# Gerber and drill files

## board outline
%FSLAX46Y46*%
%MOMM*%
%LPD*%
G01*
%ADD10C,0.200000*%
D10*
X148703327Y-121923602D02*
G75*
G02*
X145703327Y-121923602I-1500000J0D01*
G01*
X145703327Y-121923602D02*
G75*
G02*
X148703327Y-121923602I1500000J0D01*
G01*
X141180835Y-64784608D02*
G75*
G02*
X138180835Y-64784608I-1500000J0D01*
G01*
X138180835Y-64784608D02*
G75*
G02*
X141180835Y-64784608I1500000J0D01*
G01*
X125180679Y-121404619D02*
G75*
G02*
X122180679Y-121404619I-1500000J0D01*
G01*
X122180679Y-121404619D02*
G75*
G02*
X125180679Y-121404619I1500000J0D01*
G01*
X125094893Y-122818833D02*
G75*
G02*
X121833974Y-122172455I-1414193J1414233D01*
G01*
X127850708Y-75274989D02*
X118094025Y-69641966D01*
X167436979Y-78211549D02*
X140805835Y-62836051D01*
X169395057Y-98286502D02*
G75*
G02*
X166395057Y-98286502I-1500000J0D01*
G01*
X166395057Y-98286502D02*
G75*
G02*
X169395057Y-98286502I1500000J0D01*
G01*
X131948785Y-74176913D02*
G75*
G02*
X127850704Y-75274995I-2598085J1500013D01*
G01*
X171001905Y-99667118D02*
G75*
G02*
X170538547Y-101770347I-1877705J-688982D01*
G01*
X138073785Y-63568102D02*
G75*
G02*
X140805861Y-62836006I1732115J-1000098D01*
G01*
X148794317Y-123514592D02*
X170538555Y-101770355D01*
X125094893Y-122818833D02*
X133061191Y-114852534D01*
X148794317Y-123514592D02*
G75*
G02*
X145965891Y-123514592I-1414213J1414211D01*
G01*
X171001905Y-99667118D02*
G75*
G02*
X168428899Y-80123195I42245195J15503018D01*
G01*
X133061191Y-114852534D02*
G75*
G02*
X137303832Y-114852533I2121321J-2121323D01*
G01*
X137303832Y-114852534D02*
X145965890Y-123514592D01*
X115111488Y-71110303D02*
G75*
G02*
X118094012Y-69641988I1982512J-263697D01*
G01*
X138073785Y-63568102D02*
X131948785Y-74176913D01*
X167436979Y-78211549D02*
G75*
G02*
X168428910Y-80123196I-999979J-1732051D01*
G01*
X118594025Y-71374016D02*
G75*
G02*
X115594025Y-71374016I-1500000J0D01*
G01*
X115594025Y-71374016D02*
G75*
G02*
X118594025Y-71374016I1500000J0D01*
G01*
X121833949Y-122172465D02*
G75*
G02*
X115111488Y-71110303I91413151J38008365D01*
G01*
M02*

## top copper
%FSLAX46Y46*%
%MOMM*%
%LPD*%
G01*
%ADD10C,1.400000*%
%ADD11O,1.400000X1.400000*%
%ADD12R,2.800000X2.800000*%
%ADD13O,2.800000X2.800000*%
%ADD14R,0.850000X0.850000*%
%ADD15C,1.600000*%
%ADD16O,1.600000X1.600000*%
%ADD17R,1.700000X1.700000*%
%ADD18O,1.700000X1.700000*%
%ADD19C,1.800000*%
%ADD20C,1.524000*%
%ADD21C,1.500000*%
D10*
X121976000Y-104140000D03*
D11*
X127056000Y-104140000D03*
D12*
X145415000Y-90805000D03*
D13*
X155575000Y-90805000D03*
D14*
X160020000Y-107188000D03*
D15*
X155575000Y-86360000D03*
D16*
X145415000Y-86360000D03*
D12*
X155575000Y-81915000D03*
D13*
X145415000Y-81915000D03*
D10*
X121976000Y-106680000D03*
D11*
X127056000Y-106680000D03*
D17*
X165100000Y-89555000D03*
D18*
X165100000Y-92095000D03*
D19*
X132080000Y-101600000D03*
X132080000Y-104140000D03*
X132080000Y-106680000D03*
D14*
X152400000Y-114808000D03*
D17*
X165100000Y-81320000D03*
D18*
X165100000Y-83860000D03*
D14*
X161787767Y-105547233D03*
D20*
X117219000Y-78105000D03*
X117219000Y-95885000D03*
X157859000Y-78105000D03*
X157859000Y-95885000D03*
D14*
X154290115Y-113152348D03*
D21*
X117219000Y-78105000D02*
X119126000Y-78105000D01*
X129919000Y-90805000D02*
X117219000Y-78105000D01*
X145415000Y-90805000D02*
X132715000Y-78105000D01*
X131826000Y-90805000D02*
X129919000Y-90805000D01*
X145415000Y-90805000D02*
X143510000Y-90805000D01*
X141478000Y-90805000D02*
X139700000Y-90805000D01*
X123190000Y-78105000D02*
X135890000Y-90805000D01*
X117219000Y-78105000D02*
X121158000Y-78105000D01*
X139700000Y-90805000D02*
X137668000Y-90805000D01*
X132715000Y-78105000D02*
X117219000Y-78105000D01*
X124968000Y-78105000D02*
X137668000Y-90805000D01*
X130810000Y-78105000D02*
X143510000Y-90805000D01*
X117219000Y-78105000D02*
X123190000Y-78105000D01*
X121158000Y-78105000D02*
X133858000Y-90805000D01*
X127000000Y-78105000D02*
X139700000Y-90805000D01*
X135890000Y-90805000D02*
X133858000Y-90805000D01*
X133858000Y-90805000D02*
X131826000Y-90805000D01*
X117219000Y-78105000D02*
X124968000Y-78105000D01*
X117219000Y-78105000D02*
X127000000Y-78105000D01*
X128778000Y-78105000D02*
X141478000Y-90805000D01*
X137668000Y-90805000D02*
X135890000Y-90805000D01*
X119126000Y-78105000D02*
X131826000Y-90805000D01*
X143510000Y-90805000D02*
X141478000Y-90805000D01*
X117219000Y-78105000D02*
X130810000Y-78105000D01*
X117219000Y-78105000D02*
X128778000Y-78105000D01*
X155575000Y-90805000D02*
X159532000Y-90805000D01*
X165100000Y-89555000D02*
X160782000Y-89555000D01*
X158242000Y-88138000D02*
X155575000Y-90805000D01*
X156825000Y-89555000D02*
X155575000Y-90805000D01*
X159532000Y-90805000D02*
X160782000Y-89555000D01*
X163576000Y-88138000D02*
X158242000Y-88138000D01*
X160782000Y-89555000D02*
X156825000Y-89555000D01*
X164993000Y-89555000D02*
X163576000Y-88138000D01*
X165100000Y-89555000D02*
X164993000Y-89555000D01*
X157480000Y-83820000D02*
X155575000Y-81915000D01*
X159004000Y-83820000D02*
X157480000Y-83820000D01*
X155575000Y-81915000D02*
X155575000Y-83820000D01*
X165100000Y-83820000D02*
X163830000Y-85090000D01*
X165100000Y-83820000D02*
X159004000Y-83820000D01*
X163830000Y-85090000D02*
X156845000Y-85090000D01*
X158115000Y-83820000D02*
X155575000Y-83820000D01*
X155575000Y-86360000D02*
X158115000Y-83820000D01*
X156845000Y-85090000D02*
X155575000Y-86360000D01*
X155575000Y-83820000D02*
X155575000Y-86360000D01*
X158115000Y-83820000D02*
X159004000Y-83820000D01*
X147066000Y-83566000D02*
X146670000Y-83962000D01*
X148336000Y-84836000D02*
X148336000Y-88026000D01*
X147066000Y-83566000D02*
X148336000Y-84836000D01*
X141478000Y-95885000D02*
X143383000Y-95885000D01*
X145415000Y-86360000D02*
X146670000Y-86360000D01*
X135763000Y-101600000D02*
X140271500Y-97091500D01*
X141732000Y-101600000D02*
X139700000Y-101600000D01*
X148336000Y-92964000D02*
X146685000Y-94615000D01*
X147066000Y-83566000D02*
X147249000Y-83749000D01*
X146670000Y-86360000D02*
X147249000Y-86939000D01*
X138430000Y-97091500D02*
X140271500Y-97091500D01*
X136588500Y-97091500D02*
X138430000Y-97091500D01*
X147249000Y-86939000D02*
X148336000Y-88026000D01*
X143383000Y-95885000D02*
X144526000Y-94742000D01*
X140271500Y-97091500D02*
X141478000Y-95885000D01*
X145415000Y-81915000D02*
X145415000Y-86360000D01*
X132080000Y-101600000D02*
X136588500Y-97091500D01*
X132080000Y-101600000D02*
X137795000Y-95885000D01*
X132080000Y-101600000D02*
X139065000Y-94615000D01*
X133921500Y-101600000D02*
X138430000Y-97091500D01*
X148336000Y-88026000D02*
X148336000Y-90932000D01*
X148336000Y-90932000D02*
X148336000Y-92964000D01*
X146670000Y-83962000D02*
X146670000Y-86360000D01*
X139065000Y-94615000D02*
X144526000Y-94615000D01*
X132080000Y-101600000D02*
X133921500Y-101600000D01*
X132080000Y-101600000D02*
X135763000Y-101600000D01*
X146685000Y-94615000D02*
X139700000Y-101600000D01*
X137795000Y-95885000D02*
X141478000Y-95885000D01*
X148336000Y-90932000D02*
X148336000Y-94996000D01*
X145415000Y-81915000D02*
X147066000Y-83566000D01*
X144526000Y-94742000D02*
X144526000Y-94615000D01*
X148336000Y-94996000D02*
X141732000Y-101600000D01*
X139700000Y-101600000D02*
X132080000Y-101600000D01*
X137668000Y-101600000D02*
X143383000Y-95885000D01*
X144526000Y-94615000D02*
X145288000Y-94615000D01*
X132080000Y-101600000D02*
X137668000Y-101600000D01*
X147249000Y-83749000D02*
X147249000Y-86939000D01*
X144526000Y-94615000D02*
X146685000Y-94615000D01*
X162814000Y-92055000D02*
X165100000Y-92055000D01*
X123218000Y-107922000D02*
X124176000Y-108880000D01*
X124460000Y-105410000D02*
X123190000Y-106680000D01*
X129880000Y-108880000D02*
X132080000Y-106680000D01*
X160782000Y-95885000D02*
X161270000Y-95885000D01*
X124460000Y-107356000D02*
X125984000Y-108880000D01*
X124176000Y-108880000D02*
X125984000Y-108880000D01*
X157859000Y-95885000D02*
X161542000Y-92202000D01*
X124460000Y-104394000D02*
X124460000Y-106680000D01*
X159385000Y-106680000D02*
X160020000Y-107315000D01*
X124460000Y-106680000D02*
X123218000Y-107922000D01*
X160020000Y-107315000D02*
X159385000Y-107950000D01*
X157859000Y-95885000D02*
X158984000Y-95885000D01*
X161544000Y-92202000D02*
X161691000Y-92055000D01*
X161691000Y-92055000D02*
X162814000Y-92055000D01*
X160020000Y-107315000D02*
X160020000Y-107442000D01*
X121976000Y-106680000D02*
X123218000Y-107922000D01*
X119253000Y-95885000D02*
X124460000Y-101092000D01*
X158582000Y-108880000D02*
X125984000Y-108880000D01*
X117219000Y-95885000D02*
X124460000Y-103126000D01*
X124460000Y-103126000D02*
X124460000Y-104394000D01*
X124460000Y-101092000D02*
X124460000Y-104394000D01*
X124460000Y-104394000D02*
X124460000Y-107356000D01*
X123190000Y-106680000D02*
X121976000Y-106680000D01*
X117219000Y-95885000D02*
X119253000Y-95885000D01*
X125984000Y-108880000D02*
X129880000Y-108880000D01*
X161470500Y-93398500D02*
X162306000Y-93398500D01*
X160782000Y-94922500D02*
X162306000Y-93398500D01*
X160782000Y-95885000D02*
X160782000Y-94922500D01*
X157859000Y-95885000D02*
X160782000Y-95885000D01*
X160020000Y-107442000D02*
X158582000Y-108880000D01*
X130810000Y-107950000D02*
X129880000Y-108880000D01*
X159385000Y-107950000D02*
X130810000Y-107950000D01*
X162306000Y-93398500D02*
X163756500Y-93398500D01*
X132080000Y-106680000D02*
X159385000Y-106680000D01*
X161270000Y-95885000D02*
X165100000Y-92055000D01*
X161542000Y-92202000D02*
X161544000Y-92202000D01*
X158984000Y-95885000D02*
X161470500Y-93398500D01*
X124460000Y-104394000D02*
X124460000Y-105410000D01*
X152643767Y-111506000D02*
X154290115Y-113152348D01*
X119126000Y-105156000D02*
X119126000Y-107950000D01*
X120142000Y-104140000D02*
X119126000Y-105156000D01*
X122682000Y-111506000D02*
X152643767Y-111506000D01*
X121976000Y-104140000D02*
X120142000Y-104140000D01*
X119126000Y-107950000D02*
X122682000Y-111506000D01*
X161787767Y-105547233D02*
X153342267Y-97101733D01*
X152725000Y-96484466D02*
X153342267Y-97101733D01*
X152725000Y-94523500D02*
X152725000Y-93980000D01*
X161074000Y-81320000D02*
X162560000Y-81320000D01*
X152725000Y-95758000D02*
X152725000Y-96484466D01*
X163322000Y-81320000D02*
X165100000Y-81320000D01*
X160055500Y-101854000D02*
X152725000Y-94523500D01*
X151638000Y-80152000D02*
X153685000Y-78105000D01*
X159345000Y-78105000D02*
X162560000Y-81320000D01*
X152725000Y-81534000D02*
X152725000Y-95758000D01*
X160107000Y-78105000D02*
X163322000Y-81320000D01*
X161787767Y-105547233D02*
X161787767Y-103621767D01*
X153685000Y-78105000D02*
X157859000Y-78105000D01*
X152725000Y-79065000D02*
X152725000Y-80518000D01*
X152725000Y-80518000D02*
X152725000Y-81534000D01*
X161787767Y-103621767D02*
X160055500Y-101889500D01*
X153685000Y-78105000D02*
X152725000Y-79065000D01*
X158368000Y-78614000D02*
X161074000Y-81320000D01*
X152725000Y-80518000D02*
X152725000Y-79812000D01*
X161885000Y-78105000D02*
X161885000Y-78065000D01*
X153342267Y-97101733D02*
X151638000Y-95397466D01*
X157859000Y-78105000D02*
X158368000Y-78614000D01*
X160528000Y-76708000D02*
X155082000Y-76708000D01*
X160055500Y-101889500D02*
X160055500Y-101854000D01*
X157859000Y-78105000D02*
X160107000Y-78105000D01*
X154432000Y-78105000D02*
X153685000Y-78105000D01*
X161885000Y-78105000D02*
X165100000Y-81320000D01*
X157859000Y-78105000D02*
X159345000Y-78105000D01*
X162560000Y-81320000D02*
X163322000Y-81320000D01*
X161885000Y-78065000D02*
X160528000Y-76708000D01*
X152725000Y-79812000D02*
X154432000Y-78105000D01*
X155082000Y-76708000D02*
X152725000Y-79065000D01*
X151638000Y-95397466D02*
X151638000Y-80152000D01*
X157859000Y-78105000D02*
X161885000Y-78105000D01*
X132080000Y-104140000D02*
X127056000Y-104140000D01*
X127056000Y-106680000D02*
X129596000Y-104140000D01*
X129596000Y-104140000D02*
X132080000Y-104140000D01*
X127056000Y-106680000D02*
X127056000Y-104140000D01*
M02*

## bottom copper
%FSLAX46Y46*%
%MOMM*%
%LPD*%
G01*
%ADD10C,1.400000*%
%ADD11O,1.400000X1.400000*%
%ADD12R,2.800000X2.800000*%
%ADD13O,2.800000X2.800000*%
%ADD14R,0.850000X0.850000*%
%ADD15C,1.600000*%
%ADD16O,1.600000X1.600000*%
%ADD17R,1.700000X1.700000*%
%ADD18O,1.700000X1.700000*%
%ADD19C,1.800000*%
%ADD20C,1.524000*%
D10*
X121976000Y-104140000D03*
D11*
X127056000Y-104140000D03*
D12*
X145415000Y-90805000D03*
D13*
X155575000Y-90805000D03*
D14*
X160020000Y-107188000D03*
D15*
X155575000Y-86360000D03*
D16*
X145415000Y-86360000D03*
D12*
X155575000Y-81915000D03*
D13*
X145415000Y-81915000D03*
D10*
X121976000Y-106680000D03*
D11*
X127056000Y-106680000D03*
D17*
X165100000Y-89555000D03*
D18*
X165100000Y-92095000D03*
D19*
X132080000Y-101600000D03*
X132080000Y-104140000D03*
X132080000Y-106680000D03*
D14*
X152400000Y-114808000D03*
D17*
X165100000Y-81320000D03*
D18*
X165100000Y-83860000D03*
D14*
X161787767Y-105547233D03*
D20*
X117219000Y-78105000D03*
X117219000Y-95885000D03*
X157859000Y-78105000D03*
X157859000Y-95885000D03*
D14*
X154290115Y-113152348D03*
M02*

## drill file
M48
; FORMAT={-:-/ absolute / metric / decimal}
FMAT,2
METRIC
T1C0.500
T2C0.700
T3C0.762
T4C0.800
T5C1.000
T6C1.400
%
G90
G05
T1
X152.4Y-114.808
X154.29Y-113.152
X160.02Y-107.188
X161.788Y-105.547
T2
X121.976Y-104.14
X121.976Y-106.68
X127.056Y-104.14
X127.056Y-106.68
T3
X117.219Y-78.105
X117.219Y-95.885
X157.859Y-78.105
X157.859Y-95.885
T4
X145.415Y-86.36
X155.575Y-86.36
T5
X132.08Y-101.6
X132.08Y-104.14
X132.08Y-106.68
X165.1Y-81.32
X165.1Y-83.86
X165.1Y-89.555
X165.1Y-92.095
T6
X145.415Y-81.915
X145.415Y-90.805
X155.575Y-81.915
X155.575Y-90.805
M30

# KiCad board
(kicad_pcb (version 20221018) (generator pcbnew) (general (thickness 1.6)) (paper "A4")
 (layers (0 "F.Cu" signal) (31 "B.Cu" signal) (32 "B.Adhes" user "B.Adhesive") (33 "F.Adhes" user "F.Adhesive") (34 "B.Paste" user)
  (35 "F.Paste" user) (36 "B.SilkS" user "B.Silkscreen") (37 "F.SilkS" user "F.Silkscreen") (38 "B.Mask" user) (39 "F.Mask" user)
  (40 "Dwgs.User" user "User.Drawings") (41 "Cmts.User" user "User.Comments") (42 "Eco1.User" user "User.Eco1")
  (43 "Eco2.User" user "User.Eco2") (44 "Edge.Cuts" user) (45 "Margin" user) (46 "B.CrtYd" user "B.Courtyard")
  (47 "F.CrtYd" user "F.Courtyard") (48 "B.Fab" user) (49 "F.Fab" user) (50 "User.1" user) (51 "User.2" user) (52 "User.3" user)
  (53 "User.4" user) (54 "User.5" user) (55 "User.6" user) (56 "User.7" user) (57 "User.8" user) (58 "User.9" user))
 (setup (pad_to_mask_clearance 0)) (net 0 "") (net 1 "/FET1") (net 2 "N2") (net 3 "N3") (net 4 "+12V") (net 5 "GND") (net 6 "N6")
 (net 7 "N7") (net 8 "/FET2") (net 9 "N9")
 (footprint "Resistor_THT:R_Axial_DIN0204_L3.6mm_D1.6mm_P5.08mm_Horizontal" (layer "F.Cu") (at 121.976 104.14)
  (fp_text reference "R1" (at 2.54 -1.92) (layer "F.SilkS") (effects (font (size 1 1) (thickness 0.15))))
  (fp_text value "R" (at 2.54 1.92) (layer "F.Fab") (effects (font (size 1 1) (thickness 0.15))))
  (pad "1" thru_hole circle (at 0 0) (size 1.4 1.4) (drill 0.7) (layers "*.Cu" "*.Mask") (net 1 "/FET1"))
  (pad "2" thru_hole oval (at 5.08 0) (size 1.4 1.4) (drill 0.7) (layers "*.Cu" "*.Mask") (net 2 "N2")))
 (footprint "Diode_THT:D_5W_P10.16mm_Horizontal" (layer "F.Cu") (at 145.415 90.805)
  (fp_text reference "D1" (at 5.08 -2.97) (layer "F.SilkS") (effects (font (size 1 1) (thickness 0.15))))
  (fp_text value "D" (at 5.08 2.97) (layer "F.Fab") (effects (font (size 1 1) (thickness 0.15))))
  (pad "1" thru_hole rect (at 0 0) (size 2.8 2.8) (drill 1.4) (layers "*.Cu" "*.Mask") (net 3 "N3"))
  (pad "2" thru_hole oval (at 10.16 0) (size 2.8 2.8) (drill 1.4) (layers "*.Cu" "*.Mask") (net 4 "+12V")))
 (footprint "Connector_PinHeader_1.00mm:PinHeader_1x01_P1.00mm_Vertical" (layer "F.Cu") (at 160.02 107.188)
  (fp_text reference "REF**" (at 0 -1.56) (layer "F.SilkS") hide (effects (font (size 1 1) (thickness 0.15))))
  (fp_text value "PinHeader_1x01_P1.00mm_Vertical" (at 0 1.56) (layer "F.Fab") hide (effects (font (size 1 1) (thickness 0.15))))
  (pad "1" thru_hole rect (at 0 0) (size 0.85 0.85) (drill 0.5) (layers "*.Cu" "*.Mask") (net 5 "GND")))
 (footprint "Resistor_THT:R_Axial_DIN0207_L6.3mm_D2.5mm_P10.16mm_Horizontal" (layer "F.Cu") (at 155.575 86.36 180)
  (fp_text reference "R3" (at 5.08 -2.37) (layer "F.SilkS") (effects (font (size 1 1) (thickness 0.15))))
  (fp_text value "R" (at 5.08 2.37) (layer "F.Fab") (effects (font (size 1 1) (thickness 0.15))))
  (pad "1" thru_hole circle (at 0 0 180) (size 1.6 1.6) (drill 0.8) (layers "*.Cu" "*.Mask") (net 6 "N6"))
  (pad "2" thru_hole oval (at 10.16 0 180) (size 1.6 1.6) (drill 0.8) (layers "*.Cu" "*.Mask") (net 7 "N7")))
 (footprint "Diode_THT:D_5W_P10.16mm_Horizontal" (layer "F.Cu") (at 155.575 81.915 180)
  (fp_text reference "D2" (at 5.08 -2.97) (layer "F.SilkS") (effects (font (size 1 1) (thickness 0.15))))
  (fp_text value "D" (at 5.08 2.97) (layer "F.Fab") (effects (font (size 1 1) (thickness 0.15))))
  (pad "1" thru_hole rect (at 0 0 180) (size 2.8 2.8) (drill 1.4) (layers "*.Cu" "*.Mask") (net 6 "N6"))
  (pad "2" thru_hole oval (at 10.16 0 180) (size 2.8 2.8) (drill 1.4) (layers "*.Cu" "*.Mask") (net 7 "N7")))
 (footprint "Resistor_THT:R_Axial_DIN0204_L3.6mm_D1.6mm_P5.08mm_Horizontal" (layer "F.Cu") (at 121.976 106.68)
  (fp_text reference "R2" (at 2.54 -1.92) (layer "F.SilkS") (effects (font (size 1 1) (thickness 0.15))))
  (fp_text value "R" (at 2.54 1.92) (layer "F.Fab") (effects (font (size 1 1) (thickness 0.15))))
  (pad "1" thru_hole circle (at 0 0) (size 1.4 1.4) (drill 0.7) (layers "*.Cu" "*.Mask") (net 5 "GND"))
  (pad "2" thru_hole oval (at 5.08 0) (size 1.4 1.4) (drill 0.7) (layers "*.Cu" "*.Mask") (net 2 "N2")))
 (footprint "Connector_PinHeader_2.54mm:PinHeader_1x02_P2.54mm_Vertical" (layer "F.Cu") (at 165.1 89.555)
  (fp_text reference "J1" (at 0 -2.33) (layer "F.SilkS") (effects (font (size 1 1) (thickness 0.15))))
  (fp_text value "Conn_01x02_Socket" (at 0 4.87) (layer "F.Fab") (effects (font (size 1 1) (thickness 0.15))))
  (pad "1" thru_hole rect (at 0 0) (size 1.7 1.7) (drill 1) (layers "*.Cu" "*.Mask") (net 4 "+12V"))
  (pad "2" thru_hole oval (at 0 2.54) (size 1.7 1.7) (drill 1) (layers "*.Cu" "*.Mask") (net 5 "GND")))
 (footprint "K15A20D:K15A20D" (layer "F.Cu") (at 154.432 104.14 -90)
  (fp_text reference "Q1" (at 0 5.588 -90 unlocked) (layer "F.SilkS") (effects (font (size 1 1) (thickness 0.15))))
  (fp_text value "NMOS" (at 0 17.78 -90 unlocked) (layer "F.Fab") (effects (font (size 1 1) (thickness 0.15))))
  (pad "1" thru_hole circle (at -2.54 22.352 90) (size 1.8 1.8) (drill 1) (layers "*.Cu" "*.Mask") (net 7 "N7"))
  (pad "2" thru_hole circle (at 0 22.352 90) (size 1.8 1.8) (drill 1) (layers "*.Cu" "*.Mask") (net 2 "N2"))
  (pad "3" thru_hole circle (at 2.54 22.352 90) (size 1.8 1.8) (drill 1) (layers "*.Cu" "*.Mask") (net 5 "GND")))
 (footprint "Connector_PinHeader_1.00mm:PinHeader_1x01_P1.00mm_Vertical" (layer "F.Cu") (at 152.4 114.808)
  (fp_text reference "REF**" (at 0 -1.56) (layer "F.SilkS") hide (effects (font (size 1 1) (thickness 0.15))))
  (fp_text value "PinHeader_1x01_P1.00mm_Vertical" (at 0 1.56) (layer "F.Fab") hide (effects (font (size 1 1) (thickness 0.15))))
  (pad "1" thru_hole rect (at 0 0) (size 0.85 0.85) (drill 0.5) (layers "*.Cu" "*.Mask") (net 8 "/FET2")))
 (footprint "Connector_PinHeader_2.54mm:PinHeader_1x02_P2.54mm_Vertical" (layer "F.Cu") (at 165.1 81.32)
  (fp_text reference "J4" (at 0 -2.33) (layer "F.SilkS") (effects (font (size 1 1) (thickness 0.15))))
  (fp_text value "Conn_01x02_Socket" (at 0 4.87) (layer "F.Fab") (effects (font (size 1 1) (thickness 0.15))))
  (pad "1" thru_hole rect (at 0 0) (size 1.7 1.7) (drill 1) (layers "*.Cu" "*.Mask") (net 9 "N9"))
  (pad "2" thru_hole oval (at 0 2.54) (size 1.7 1.7) (drill 1) (layers "*.Cu" "*.Mask") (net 6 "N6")))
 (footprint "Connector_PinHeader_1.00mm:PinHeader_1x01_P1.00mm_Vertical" (layer "F.Cu") (at 161.787767 105.547233)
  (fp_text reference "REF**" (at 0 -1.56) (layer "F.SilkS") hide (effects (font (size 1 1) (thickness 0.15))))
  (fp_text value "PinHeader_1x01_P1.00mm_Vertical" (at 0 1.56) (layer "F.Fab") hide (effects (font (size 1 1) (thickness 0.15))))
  (pad "1" thru_hole rect (at 0 0) (size 0.85 0.85) (drill 0.5) (layers "*.Cu" "*.Mask") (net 9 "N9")))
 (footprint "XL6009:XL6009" (layer "F.Cu") (at 112.139 86.995 90)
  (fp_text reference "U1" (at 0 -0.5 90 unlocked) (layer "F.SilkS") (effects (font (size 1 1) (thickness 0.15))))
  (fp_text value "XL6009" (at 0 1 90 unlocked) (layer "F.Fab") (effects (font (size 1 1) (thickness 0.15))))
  (pad "1" thru_hole circle (at 8.89 5.08 90) (size 1.524 1.524) (drill 0.762) (layers "*.Cu" "*.Mask") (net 3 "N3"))
  (pad "2" thru_hole circle (at -8.89 5.08 90) (size 1.524 1.524) (drill 0.762) (layers "*.Cu" "*.Mask") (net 5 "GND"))
  (pad "3" thru_hole circle (at 8.89 45.72 90) (size 1.524 1.524) (drill 0.762) (layers "*.Cu" "*.Mask") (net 9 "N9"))
  (pad "4" thru_hole circle (at -8.89 45.72 90) (size 1.524 1.524) (drill 0.762) (layers "*.Cu" "*.Mask") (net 5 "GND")))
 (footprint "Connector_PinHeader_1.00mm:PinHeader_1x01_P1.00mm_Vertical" (layer "F.Cu") (at 154.290115 113.152348)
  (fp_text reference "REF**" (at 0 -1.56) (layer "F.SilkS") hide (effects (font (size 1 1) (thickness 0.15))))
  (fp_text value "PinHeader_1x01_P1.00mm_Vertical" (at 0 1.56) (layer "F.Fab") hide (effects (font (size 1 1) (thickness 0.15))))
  (pad "1" thru_hole rect (at 0 0) (size 0.85 0.85) (drill 0.5) (layers "*.Cu" "*.Mask") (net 1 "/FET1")))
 (gr_circle (center 147.203327 121.923602) (end 145.703327 121.923602) (stroke (width 0.2) (type solid)) (fill none) (layer "Edge.Cuts"))
 (gr_circle (center 139.680835 64.784608) (end 138.180835 64.784608) (stroke (width 0.2) (type solid)) (fill none) (layer "Edge.Cuts"))
 (gr_circle (center 123.680679 121.404619) (end 122.180679 121.404619) (stroke (width 0.2) (type solid)) (fill none) (layer "Edge.Cuts"))
 (gr_arc (start 125.094893 122.818833) (mid 123.291827 123.366429) (end 121.833949 122.172465) (stroke (width 0.2) (type solid))
  (layer "Edge.Cuts"))
 (gr_line (start 127.850708 75.274989) (end 118.094025 69.641966) (stroke (width 0.2) (type solid)) (layer "Edge.Cuts"))
 (gr_line (start 167.436979 78.211549) (end 140.805835 62.836051) (stroke (width 0.2) (type solid)) (layer "Edge.Cuts"))
 (gr_circle (center 167.895057 98.286502) (end 166.395057 98.286502) (stroke (width 0.2) (type solid)) (fill none) (layer "Edge.Cuts"))
 (gr_arc (start 131.948785 74.176913) (mid 130.127164 75.57469) (end 127.850708 75.274989) (stroke (width 0.2) (type solid))
  (layer "Edge.Cuts"))
 (gr_arc (start 171.001905 99.667118) (mid 171.077482 100.78642) (end 170.538555 101.770355) (stroke (width 0.2) (type solid))
  (layer "Edge.Cuts"))
 (gr_arc (start 138.073785 63.568102) (mid 139.288193 62.636273) (end 140.805835 62.836051) (stroke (width 0.2) (type solid))
  (layer "Edge.Cuts"))
 (gr_line (start 148.794317 123.514592) (end 170.538555 101.770355) (stroke (width 0.2) (type solid)) (layer "Edge.Cuts"))
 (gr_line (start 125.094893 122.818833) (end 133.061191 114.852534) (stroke (width 0.2) (type solid)) (layer "Edge.Cuts"))
 (gr_arc (start 148.794317 123.514592) (mid 147.380103 124.100379) (end 145.96589 123.514592) (stroke (width 0.2) (type solid))
  (layer "Edge.Cuts"))
 (gr_arc (start 171.001905 99.667118) (mid 168.632081 90.037778) (end 168.428899 80.123195) (stroke (width 0.2) (type solid))
  (layer "Edge.Cuts"))
 (gr_arc (start 133.061191 114.852534) (mid 135.182511 113.973855) (end 137.303832 114.852534) (stroke (width 0.2) (type solid))
  (layer "Edge.Cuts"))
 (gr_line (start 137.303832 114.852534) (end 145.96589 123.514592) (stroke (width 0.2) (type solid)) (layer "Edge.Cuts"))
 (gr_arc (start 115.111488 71.110303) (mid 116.210646 69.579682) (end 118.094025 69.641966) (stroke (width 0.2) (type solid))
  (layer "Edge.Cuts"))
 (gr_line (start 138.073785 63.568102) (end 131.948785 74.176913) (stroke (width 0.2) (type solid)) (layer "Edge.Cuts"))
 (gr_arc (start 167.436979 78.211549) (mid 168.212232 79.022454) (end 168.428899 80.123195) (stroke (width 0.2) (type solid))
  (layer "Edge.Cuts"))
 (gr_circle (center 117.094025 71.374016) (end 115.594025 71.374016) (stroke (width 0.2) (type solid)) (fill none) (layer "Edge.Cuts"))
 (gr_arc (start 121.833949 122.172465) (mid 115.094059 97.086193) (end 115.111488 71.110303) (stroke (width 0.2) (type solid))
  (layer "Edge.Cuts"))
 (segment (start 117.219 78.105) (end 119.126 78.105) (width 1.5) (layer "F.Cu") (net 3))
 (segment (start 129.919 90.805) (end 117.219 78.105) (width 1.5) (layer "F.Cu") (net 3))
 (segment (start 145.415 90.805) (end 132.715 78.105) (width 1.5) (layer "F.Cu") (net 3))
 (segment (start 131.826 90.805) (end 129.919 90.805) (width 1.5) (layer "F.Cu") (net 3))
 (segment (start 145.415 90.805) (end 143.51 90.805) (width 1.5) (layer "F.Cu") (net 3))
 (segment (start 141.478 90.805) (end 139.7 90.805) (width 1.5) (layer "F.Cu") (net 3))
 (segment (start 123.19 78.105) (end 135.89 90.805) (width 1.5) (layer "F.Cu") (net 3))
 (segment (start 117.219 78.105) (end 121.158 78.105) (width 1.5) (layer "F.Cu") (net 3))
 (segment (start 139.7 90.805) (end 137.668 90.805) (width 1.5) (layer "F.Cu") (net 3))
 (segment (start 132.715 78.105) (end 117.219 78.105) (width 1.5) (layer "F.Cu") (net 3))
 (segment (start 124.968 78.105) (end 137.668 90.805) (width 1.5) (layer "F.Cu") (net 3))
 (segment (start 130.81 78.105) (end 143.51 90.805) (width 1.5) (layer "F.Cu") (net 3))
 (segment (start 117.219 78.105) (end 123.19 78.105) (width 1.5) (layer "F.Cu") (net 3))
 (segment (start 121.158 78.105) (end 133.858 90.805) (width 1.5) (layer "F.Cu") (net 3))
 (segment (start 127 78.105) (end 139.7 90.805) (width 1.5) (layer "F.Cu") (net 3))
 (segment (start 135.89 90.805) (end 133.858 90.805) (width 1.5) (layer "F.Cu") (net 3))
 (segment (start 133.858 90.805) (end 131.826 90.805) (width 1.5) (layer "F.Cu") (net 3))
 (segment (start 117.219 78.105) (end 124.968 78.105) (width 1.5) (layer "F.Cu") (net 3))
 (segment (start 117.219 78.105) (end 127 78.105) (width 1.5) (layer "F.Cu") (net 3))
 (segment (start 128.778 78.105) (end 141.478 90.805) (width 1.5) (layer "F.Cu") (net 3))
 (segment (start 137.668 90.805) (end 135.89 90.805) (width 1.5) (layer "F.Cu") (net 3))
 (segment (start 119.126 78.105) (end 131.826 90.805) (width 1.5) (layer "F.Cu") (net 3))
 (segment (start 143.51 90.805) (end 141.478 90.805) (width 1.5) (layer "F.Cu") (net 3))
 (segment (start 117.219 78.105) (end 130.81 78.105) (width 1.5) (layer "F.Cu") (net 3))
 (segment (start 117.219 78.105) (end 128.778 78.105) (width 1.5) (layer "F.Cu") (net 3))
 (segment (start 155.575 90.805) (end 159.532 90.805) (width 1.5) (layer "F.Cu") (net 4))
 (segment (start 165.1 89.555) (end 160.782 89.555) (width 1.5) (layer "F.Cu") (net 4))
 (segment (start 158.242 88.138) (end 155.575 90.805) (width 1.5) (layer "F.Cu") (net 4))
 (segment (start 156.825 89.555) (end 155.575 90.805) (width 1.5) (layer "F.Cu") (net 4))
 (segment (start 159.532 90.805) (end 160.782 89.555) (width 1.5) (layer "F.Cu") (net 4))
 (segment (start 163.576 88.138) (end 158.242 88.138) (width 1.5) (layer "F.Cu") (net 4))
 (segment (start 160.782 89.555) (end 156.825 89.555) (width 1.5) (layer "F.Cu") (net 4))
 (segment (start 164.993 89.555) (end 163.576 88.138) (width 1.5) (layer "F.Cu") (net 4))
 (segment (start 165.1 89.555) (end 164.993 89.555) (width 1.5) (layer "F.Cu") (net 4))
 (segment (start 157.48 83.82) (end 155.575 81.915) (width 1.5) (layer "F.Cu") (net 6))
 (segment (start 159.004 83.82) (end 157.48 83.82) (width 1.5) (layer "F.Cu") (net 6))
 (segment (start 155.575 81.915) (end 155.575 83.82) (width 1.5) (layer "F.Cu") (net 6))
 (segment (start 165.1 83.82) (end 163.83 85.09) (width 1.5) (layer "F.Cu") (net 6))
 (segment (start 165.1 83.82) (end 159.004 83.82) (width 1.5) (layer "F.Cu") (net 6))
 (segment (start 163.83 85.09) (end 156.845 85.09) (width 1.5) (layer "F.Cu") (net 6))
 (segment (start 158.115 83.82) (end 155.575 83.82) (width 1.5) (layer "F.Cu") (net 6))
 (segment (start 155.575 86.36) (end 158.115 83.82) (width 1.5) (layer "F.Cu") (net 6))
 (segment (start 156.845 85.09) (end 155.575 86.36) (width 1.5) (layer "F.Cu") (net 6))
 (segment (start 155.575 83.82) (end 155.575 86.36) (width 1.5) (layer "F.Cu") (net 6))
 (segment (start 158.115 83.82) (end 159.004 83.82) (width 1.5) (layer "F.Cu") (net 6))
 (segment (start 147.066 83.566) (end 146.67 83.962) (width 1.5) (layer "F.Cu") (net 7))
 (segment (start 148.336 84.836) (end 148.336 88.026) (width 1.5) (layer "F.Cu") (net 7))
 (segment (start 147.066 83.566) (end 148.336 84.836) (width 1.5) (layer "F.Cu") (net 7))
 (segment (start 141.478 95.885) (end 143.383 95.885) (width 1.5) (layer "F.Cu") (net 7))
 (segment (start 145.415 86.36) (end 146.67 86.36) (width 1.5) (layer "F.Cu") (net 7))
 (segment (start 135.763 101.6) (end 140.2715 97.0915) (width 1.5) (layer "F.Cu") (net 7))
 (segment (start 141.732 101.6) (end 139.7 101.6) (width 1.5) (layer "F.Cu") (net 7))
 (segment (start 148.336 92.964) (end 146.685 94.615) (width 1.5) (layer "F.Cu") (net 7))
 (segment (start 147.066 83.566) (end 147.249 83.749) (width 1.5) (layer "F.Cu") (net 7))
 (segment (start 146.67 86.36) (end 147.249 86.939) (width 1.5) (layer "F.Cu") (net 7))
 (segment (start 138.43 97.0915) (end 140.2715 97.0915) (width 1.5) (layer "F.Cu") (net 7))
 (segment (start 136.5885 97.0915) (end 138.43 97.0915) (width 1.5) (layer "F.Cu") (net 7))
 (segment (start 147.249 86.939) (end 148.336 88.026) (width 1.5) (layer "F.Cu") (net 7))
 (segment (start 143.383 95.885) (end 144.526 94.742) (width 1.5) (layer "F.Cu") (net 7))
 (segment (start 140.2715 97.0915) (end 141.478 95.885) (width 1.5) (layer "F.Cu") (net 7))
 (segment (start 145.415 81.915) (end 145.415 86.36) (width 1.5) (layer "F.Cu") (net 7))
 (segment (start 132.08 101.6) (end 136.5885 97.0915) (width 1.5) (layer "F.Cu") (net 7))
 (segment (start 132.08 101.6) (end 137.795 95.885) (width 1.5) (layer "F.Cu") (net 7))
 (segment (start 132.08 101.6) (end 139.065 94.615) (width 1.5) (layer "F.Cu") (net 7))
 (segment (start 133.9215 101.6) (end 138.43 97.0915) (width 1.5) (layer "F.Cu") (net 7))
 (segment (start 148.336 88.026) (end 148.336 90.932) (width 1.5) (layer "F.Cu") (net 7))
 (segment (start 148.336 90.932) (end 148.336 92.964) (width 1.5) (layer "F.Cu") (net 7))
 (segment (start 146.67 83.962) (end 146.67 86.36) (width 1.5) (layer "F.Cu") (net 7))
 (segment (start 139.065 94.615) (end 144.526 94.615) (width 1.5) (layer "F.Cu") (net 7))
 (segment (start 132.08 101.6) (end 133.9215 101.6) (width 1.5) (layer "F.Cu") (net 7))
 (segment (start 132.08 101.6) (end 135.763 101.6) (width 1.5) (layer "F.Cu") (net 7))
 (segment (start 146.685 94.615) (end 139.7 101.6) (width 1.5) (layer "F.Cu") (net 7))
 (segment (start 137.795 95.885) (end 141.478 95.885) (width 1.5) (layer "F.Cu") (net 7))
 (segment (start 148.336 90.932) (end 148.336 94.996) (width 1.5) (layer "F.Cu") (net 7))
 (segment (start 145.415 81.915) (end 147.066 83.566) (width 1.5) (layer "F.Cu") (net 7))
 (segment (start 144.526 94.742) (end 144.526 94.615) (width 1.5) (layer "F.Cu") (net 7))
 (segment (start 148.336 94.996) (end 141.732 101.6) (width 1.5) (layer "F.Cu") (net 7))
 (segment (start 139.7 101.6) (end 132.08 101.6) (width 1.5) (layer "F.Cu") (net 7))
 (segment (start 137.668 101.6) (end 143.383 95.885) (width 1.5) (layer "F.Cu") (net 7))
 (segment (start 144.526 94.615) (end 145.288 94.615) (width 1.5) (layer "F.Cu") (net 7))
 (segment (start 132.08 101.6) (end 137.668 101.6) (width 1.5) (layer "F.Cu") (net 7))
 (segment (start 147.249 83.749) (end 147.249 86.939) (width 1.5) (layer "F.Cu") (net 7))
 (segment (start 144.526 94.615) (end 146.685 94.615) (width 1.5) (layer "F.Cu") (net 7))
 (segment (start 162.814 92.055) (end 165.1 92.055) (width 1.5) (layer "F.Cu") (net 5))
 (segment (start 123.218 107.922) (end 124.176 108.88) (width 1.5) (layer "F.Cu") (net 5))
 (segment (start 124.46 105.41) (end 123.19 106.68) (width 1.5) (layer "F.Cu") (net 5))
 (segment (start 129.88 108.88) (end 132.08 106.68) (width 1.5) (layer "F.Cu") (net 5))
 (segment (start 160.782 95.885) (end 161.27 95.885) (width 1.5) (layer "F.Cu") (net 5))
 (segment (start 124.46 107.356) (end 125.984 108.88) (width 1.5) (layer "F.Cu") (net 5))
 (segment (start 124.176 108.88) (end 125.984 108.88) (width 1.5) (layer "F.Cu") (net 5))
 (segment (start 157.859 95.885) (end 161.542 92.202) (width 1.5) (layer "F.Cu") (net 5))
 (segment (start 124.46 104.394) (end 124.46 106.68) (width 1.5) (layer "F.Cu") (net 5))
 (segment (start 159.385 106.68) (end 160.02 107.315) (width 1.5) (layer "F.Cu") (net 5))
 (segment (start 124.46 106.68) (end 123.218 107.922) (width 1.5) (layer "F.Cu") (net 5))
 (segment (start 160.02 107.315) (end 159.385 107.95) (width 1.5) (layer "F.Cu") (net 5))
 (segment (start 157.859 95.885) (end 158.984 95.885) (width 1.5) (layer "F.Cu") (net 5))
 (segment (start 161.544 92.202) (end 161.691 92.055) (width 1.5) (layer "F.Cu") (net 5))
 (segment (start 161.691 92.055) (end 162.814 92.055) (width 1.5) (layer "F.Cu") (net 5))
 (segment (start 160.02 107.315) (end 160.02 107.442) (width 1.5) (layer "F.Cu") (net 5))
 (segment (start 121.976 106.68) (end 123.218 107.922) (width 1.5) (layer "F.Cu") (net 5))
 (segment (start 119.253 95.885) (end 124.46 101.092) (width 1.5) (layer "F.Cu") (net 5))
 (segment (start 158.582 108.88) (end 125.984 108.88) (width 1.5) (layer "F.Cu") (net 5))
 (segment (start 117.219 95.885) (end 124.46 103.126) (width 1.5) (layer "F.Cu") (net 5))
 (segment (start 124.46 103.126) (end 124.46 104.394) (width 1.5) (layer "F.Cu") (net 5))
 (segment (start 124.46 101.092) (end 124.46 104.394) (width 1.5) (layer "F.Cu") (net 5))
 (segment (start 124.46 104.394) (end 124.46 107.356) (width 1.5) (layer "F.Cu") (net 5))
 (segment (start 123.19 106.68) (end 121.976 106.68) (width 1.5) (layer "F.Cu") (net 5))
 (segment (start 117.219 95.885) (end 119.253 95.885) (width 1.5) (layer "F.Cu") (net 5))
 (segment (start 125.984 108.88) (end 129.88 108.88) (width 1.5) (layer "F.Cu") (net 5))
 (segment (start 161.4705 93.3985) (end 162.306 93.3985) (width 1.5) (layer "F.Cu") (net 5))
 (segment (start 160.782 94.9225) (end 162.306 93.3985) (width 1.5) (layer "F.Cu") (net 5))
 (segment (start 160.782 95.885) (end 160.782 94.9225) (width 1.5) (layer "F.Cu") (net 5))
 (segment (start 157.859 95.885) (end 160.782 95.885) (width 1.5) (layer "F.Cu") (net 5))
 (segment (start 160.02 107.442) (end 158.582 108.88) (width 1.5) (layer "F.Cu") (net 5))
 (segment (start 130.81 107.95) (end 129.88 108.88) (width 1.5) (layer "F.Cu") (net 5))
 (segment (start 159.385 107.95) (end 130.81 107.95) (width 1.5) (layer "F.Cu") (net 5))
 (segment (start 162.306 93.3985) (end 163.7565 93.3985) (width 1.5) (layer "F.Cu") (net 5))
 (segment (start 132.08 106.68) (end 159.385 106.68) (width 1.5) (layer "F.Cu") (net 5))
 (segment (start 161.27 95.885) (end 165.1 92.055) (width 1.5) (layer "F.Cu") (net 5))
 (segment (start 161.542 92.202) (end 161.544 92.202) (width 1.5) (layer "F.Cu") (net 5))
 (segment (start 158.984 95.885) (end 161.4705 93.3985) (width 1.5) (layer "F.Cu") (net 5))
 (segment (start 124.46 104.394) (end 124.46 105.41) (width 1.5) (layer "F.Cu") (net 5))
 (segment (start 152.643767 111.506) (end 154.290115 113.152348) (width 1.5) (layer "F.Cu") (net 1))
 (segment (start 119.126 105.156) (end 119.126 107.95) (width 1.5) (layer "F.Cu") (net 1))
 (segment (start 120.142 104.14) (end 119.126 105.156) (width 1.5) (layer "F.Cu") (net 1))
 (segment (start 122.682 111.506) (end 152.643767 111.506) (width 1.5) (layer "F.Cu") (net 1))
 (segment (start 121.976 104.14) (end 120.142 104.14) (width 1.5) (layer "F.Cu") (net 1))
 (segment (start 119.126 107.95) (end 122.682 111.506) (width 1.5) (layer "F.Cu") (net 1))
 (segment (start 161.787767 105.547233) (end 153.342267 97.101733) (width 1.5) (layer "F.Cu") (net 9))
 (segment (start 152.725 96.484466) (end 153.342267 97.101733) (width 1.5) (layer "F.Cu") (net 9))
 (segment (start 152.725 94.5235) (end 152.725 93.98) (width 1.5) (layer "F.Cu") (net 9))
 (segment (start 161.074 81.32) (end 162.56 81.32) (width 1.5) (layer "F.Cu") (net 9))
 (segment (start 152.725 95.758) (end 152.725 96.484466) (width 1.5) (layer "F.Cu") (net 9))
 (segment (start 163.322 81.32) (end 165.1 81.32) (width 1.5) (layer "F.Cu") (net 9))
 (segment (start 160.0555 101.854) (end 152.725 94.5235) (width 1.5) (layer "F.Cu") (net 9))
 (segment (start 151.638 80.152) (end 153.685 78.105) (width 1.5) (layer "F.Cu") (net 9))
 (segment (start 159.345 78.105) (end 162.56 81.32) (width 1.5) (layer "F.Cu") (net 9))
 (segment (start 152.725 81.534) (end 152.725 95.758) (width 1.5) (layer "F.Cu") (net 9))
 (segment (start 160.107 78.105) (end 163.322 81.32) (width 1.5) (layer "F.Cu") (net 9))
 (segment (start 161.787767 105.547233) (end 161.787767 103.621767) (width 1.5) (layer "F.Cu") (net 9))
 (segment (start 153.685 78.105) (end 157.859 78.105) (width 1.5) (layer "F.Cu") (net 9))
 (segment (start 152.725 79.065) (end 152.725 80.518) (width 1.5) (layer "F.Cu") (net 9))
 (segment (start 152.725 80.518) (end 152.725 81.534) (width 1.5) (layer "F.Cu") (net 9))
 (segment (start 161.787767 103.621767) (end 160.0555 101.8895) (width 1.5) (layer "F.Cu") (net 9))
 (segment (start 153.685 78.105) (end 152.725 79.065) (width 1.5) (layer "F.Cu") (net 9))
 (segment (start 158.368 78.614) (end 161.074 81.32) (width 1.5) (layer "F.Cu") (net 9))
 (segment (start 152.725 80.518) (end 152.725 79.812) (width 1.5) (layer "F.Cu") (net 9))
 (segment (start 161.885 78.105) (end 161.885 78.065) (width 1.5) (layer "F.Cu") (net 9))
 (segment (start 153.342267 97.101733) (end 151.638 95.397466) (width 1.5) (layer "F.Cu") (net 9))
 (segment (start 157.859 78.105) (end 158.368 78.614) (width 1.5) (layer "F.Cu") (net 9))
 (segment (start 160.528 76.708) (end 155.082 76.708) (width 1.5) (layer "F.Cu") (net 9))
 (segment (start 160.0555 101.8895) (end 160.0555 101.854) (width 1.5) (layer "F.Cu") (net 9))
 (segment (start 157.859 78.105) (end 160.107 78.105) (width 1.5) (layer "F.Cu") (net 9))
 (segment (start 154.432 78.105) (end 153.685 78.105) (width 1.5) (layer "F.Cu") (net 9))
 (segment (start 161.885 78.105) (end 165.1 81.32) (width 1.5) (layer "F.Cu") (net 9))
 (segment (start 157.859 78.105) (end 159.345 78.105) (width 1.5) (layer "F.Cu") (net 9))
 (segment (start 162.56 81.32) (end 163.322 81.32) (width 1.5) (layer "F.Cu") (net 9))
 (segment (start 161.885 78.065) (end 160.528 76.708) (width 1.5) (layer "F.Cu") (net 9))
 (segment (start 152.725 79.812) (end 154.432 78.105) (width 1.5) (layer "F.Cu") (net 9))
 (segment (start 155.082 76.708) (end 152.725 79.065) (width 1.5) (layer "F.Cu") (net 9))
 (segment (start 151.638 95.397466) (end 151.638 80.152) (width 1.5) (layer "F.Cu") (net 9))
 (segment (start 157.859 78.105) (end 161.885 78.105) (width 1.5) (layer "F.Cu") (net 9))
 (segment (start 132.08 104.14) (end 127.056 104.14) (width 1.5) (layer "F.Cu") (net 2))
 (segment (start 127.056 106.68) (end 129.596 104.14) (width 1.5) (layer "F.Cu") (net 2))
 (segment (start 129.596 104.14) (end 132.08 104.14) (width 1.5) (layer "F.Cu") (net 2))
 (segment (start 127.056 106.68) (end 127.056 104.14) (width 1.5) (layer "F.Cu") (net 2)))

